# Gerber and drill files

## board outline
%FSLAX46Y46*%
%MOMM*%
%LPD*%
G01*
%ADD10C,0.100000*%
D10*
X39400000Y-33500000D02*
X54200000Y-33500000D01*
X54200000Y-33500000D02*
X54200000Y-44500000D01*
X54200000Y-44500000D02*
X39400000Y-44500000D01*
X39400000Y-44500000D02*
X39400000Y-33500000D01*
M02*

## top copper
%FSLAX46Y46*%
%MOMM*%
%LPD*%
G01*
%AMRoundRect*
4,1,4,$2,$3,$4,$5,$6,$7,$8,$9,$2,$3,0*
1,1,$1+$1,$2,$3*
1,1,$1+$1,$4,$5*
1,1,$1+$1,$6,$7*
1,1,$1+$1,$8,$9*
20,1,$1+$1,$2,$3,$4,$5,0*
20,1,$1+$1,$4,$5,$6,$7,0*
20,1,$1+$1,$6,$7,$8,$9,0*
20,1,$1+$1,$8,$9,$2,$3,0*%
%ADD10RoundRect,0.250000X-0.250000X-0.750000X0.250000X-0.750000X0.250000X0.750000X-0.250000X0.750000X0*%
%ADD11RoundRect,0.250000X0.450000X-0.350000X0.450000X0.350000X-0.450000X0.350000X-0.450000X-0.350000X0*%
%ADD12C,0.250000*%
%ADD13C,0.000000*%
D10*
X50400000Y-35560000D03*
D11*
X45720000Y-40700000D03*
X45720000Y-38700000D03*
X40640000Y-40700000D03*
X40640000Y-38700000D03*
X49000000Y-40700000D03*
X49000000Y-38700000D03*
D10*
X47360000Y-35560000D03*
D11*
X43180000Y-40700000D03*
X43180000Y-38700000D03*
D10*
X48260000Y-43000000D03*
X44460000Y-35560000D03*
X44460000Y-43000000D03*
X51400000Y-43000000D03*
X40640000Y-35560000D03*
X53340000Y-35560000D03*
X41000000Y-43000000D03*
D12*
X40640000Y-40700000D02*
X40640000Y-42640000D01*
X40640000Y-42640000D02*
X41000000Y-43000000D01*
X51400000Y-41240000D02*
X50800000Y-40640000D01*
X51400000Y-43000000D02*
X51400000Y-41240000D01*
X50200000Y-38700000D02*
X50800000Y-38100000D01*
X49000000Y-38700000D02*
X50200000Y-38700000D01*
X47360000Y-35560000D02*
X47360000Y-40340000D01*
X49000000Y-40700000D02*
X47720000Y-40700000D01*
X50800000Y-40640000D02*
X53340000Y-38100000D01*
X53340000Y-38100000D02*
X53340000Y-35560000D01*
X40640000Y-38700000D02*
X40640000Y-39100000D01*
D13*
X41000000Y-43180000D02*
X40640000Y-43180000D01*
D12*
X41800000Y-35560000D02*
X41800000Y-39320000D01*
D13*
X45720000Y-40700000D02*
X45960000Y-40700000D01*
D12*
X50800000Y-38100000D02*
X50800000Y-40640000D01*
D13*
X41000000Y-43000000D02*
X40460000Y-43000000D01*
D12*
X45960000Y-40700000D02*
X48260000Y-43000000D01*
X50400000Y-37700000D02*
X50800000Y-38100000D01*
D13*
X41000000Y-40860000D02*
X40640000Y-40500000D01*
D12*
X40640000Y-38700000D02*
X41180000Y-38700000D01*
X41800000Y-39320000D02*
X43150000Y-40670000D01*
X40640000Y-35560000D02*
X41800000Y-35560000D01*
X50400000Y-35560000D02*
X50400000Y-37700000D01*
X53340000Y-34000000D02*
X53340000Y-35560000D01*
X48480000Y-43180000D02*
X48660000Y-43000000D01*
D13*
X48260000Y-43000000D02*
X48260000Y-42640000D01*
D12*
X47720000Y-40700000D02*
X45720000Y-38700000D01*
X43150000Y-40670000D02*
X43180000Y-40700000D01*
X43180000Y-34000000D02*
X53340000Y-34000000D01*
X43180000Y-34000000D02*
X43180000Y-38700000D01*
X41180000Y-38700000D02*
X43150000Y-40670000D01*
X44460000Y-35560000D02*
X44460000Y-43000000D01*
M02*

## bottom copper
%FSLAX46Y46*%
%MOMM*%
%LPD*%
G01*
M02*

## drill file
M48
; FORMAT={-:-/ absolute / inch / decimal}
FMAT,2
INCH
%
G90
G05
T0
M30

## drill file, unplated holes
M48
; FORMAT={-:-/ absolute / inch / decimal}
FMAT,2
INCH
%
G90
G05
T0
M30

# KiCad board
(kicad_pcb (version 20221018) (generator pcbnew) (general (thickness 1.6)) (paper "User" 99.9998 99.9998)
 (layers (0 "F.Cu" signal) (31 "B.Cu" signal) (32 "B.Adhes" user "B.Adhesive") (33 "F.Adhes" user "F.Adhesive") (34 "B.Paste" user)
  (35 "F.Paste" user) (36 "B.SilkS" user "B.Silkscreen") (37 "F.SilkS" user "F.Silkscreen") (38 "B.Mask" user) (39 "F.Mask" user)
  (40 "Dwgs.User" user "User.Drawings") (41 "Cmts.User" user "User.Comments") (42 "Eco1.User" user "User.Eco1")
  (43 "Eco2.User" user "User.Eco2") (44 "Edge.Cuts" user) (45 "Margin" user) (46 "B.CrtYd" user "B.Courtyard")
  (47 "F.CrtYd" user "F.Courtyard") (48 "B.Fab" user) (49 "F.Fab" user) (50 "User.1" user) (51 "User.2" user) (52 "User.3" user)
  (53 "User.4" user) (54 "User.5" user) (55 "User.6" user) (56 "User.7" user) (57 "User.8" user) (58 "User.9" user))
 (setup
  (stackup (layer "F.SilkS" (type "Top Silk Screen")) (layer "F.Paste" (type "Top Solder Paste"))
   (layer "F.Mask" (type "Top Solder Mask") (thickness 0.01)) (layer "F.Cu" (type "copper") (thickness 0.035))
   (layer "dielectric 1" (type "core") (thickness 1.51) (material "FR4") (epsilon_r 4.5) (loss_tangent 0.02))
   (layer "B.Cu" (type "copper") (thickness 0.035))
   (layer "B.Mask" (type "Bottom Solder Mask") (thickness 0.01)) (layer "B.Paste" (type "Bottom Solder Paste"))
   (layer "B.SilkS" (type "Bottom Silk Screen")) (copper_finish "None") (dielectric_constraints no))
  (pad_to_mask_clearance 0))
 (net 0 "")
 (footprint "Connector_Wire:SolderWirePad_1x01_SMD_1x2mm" (layer "F.Cu") (at 50.4 35.56)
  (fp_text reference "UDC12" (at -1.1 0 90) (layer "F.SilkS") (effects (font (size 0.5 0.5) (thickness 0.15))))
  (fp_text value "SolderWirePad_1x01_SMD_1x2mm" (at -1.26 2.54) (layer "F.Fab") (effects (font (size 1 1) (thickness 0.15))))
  (pad "1" smd roundrect (at 0 0) (size 1 2) (layers "F.Cu" "F.Paste" "F.Mask") (roundrect_rratio 0.25)))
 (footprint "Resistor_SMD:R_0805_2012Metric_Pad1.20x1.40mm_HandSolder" (layer "F.Cu") (at 45.72 39.7 90)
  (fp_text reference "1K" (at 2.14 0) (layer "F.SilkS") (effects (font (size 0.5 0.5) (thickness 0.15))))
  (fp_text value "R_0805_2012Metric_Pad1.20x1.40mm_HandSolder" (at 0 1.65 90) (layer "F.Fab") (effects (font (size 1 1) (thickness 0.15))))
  (pad "1" smd roundrect (at -1 0 90) (size 1.2 1.4) (layers "F.Cu" "F.Paste" "F.Mask") (roundrect_rratio 0.2083333333))
  (pad "2" smd roundrect (at 1 0 90) (size 1.2 1.4) (layers "F.Cu" "F.Paste" "F.Mask") (roundrect_rratio 0.2083333333)))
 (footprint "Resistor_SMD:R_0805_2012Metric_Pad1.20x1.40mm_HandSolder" (layer "F.Cu") (at 40.64 39.7 90)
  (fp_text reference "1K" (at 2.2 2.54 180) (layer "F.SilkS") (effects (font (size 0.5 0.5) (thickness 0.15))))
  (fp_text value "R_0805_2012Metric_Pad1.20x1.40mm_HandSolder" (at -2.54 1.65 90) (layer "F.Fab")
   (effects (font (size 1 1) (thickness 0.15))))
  (pad "1" smd roundrect (at -1 0 90) (size 1.2 1.4) (layers "F.Cu" "F.Paste" "F.Mask") (roundrect_rratio 0.2083333333))
  (pad "2" smd roundrect (at 1 0 90) (size 1.2 1.4) (layers "F.Cu" "F.Paste" "F.Mask") (roundrect_rratio 0.2083333333)))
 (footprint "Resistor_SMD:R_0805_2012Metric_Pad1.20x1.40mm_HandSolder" (layer "F.Cu") (at 49 39.7 90)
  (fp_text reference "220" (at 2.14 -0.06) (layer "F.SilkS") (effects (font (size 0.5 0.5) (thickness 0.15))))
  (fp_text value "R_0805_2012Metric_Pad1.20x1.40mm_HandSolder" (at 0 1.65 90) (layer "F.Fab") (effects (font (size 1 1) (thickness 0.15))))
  (pad "1" smd roundrect (at -1 0 90) (size 1.2 1.4) (layers "F.Cu" "F.Paste" "F.Mask") (roundrect_rratio 0.2083333333))
  (pad "2" smd roundrect (at 1 0 90) (size 1.2 1.4) (layers "F.Cu" "F.Paste" "F.Mask") (roundrect_rratio 0.2083333333)))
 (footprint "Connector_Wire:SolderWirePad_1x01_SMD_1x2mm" (layer "F.Cu") (at 47.36 35.56)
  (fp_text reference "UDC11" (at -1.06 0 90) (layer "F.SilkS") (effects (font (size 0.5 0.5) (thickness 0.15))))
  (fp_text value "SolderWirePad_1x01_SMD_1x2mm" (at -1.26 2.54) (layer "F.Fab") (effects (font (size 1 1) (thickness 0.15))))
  (pad "1" smd roundrect (at 0 0) (size 1 2) (layers "F.Cu" "F.Paste" "F.Mask") (roundrect_rratio 0.25)))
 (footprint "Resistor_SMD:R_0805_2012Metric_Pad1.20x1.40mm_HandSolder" (layer "F.Cu") (at 43.18 39.7 90)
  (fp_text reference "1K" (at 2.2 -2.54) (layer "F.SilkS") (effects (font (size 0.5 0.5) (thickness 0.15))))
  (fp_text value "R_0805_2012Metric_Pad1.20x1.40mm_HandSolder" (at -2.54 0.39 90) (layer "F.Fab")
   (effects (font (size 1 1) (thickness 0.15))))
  (pad "1" smd roundrect (at -1 0 90) (size 1.2 1.4) (layers "F.Cu" "F.Paste" "F.Mask") (roundrect_rratio 0.2083333333))
  (pad "2" smd roundrect (at 1 0 90) (size 1.2 1.4) (layers "F.Cu" "F.Paste" "F.Mask") (roundrect_rratio 0.2083333333)))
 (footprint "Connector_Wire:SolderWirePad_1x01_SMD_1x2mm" (layer "F.Cu") (at 48.26 43)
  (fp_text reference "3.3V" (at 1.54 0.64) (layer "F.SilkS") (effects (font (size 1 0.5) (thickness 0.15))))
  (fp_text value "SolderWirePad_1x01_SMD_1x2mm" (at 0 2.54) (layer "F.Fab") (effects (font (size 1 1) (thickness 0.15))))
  (pad "1" smd roundrect (at 0 0) (size 1 2) (layers "F.Cu" "F.Paste" "F.Mask") (roundrect_rratio 0.25)))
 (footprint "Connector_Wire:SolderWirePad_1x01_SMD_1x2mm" (layer "F.Cu") (at 44.46 35.56)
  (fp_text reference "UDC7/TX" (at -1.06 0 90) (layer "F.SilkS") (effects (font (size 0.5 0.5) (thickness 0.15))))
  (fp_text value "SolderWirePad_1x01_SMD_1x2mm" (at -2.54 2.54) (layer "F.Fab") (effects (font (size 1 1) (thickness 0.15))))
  (pad "1" smd roundrect (at 0 0) (size 1 2) (layers "F.Cu" "F.Paste" "F.Mask") (roundrect_rratio 0.25)))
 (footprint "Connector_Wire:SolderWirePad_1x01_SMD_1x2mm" (layer "F.Cu") (at 44.46 43)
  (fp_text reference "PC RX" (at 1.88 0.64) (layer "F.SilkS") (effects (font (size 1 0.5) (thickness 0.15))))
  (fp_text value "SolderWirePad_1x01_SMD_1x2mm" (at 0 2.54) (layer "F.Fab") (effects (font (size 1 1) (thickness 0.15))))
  (pad "1" smd roundrect (at 0 0) (size 1 2) (layers "F.Cu" "F.Paste" "F.Mask") (roundrect_rratio 0.25)))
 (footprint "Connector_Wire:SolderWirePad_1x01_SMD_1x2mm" (layer "F.Cu") (at 51.4 43)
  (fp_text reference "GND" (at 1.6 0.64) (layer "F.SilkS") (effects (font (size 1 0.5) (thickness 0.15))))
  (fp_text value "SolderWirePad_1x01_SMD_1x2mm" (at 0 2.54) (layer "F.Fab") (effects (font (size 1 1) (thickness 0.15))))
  (pad "1" smd roundrect (at 0 0) (size 1 2) (layers "F.Cu" "F.Paste" "F.Mask") (roundrect_rratio 0.25)))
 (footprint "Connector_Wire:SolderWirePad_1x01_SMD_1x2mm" (layer "F.Cu") (at 40.64 35.56)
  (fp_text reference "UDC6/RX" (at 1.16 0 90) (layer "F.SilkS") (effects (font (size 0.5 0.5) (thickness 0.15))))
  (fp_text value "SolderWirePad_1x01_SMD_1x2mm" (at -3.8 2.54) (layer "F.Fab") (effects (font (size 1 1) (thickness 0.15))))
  (pad "1" smd roundrect (at 0 0) (size 1 2) (layers "F.Cu" "F.Paste" "F.Mask") (roundrect_rratio 0.25)))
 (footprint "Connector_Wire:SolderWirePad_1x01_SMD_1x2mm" (layer "F.Cu") (at 53.34 35.56)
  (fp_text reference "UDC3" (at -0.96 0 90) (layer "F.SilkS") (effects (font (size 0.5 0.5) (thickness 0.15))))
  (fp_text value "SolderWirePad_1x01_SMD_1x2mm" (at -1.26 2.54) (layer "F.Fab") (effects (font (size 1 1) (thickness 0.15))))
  (pad "1" smd roundrect (at 0 0) (size 1 2) (layers "F.Cu" "F.Paste" "F.Mask") (roundrect_rratio 0.25)))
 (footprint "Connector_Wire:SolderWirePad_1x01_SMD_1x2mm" (layer "F.Cu") (at 41 43)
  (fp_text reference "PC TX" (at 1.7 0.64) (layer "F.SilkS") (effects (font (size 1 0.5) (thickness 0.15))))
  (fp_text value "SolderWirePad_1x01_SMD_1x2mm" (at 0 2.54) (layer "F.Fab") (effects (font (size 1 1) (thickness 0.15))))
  (pad "1" smd roundrect (at 0 0) (size 1 2) (layers "F.Cu" "F.Paste" "F.Mask") (roundrect_rratio 0.25)))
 (gr_rect (start 39.4 33.5) (end 54.2 44.5) (stroke (width 0.1) (type default)) (fill none) (layer "Edge.Cuts"))
 (segment (start 51.4 43) (end 51.4 41.24) (width 0.25) (layer "F.Cu") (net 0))
 (segment (start 47.36 35.56) (end 47.36 40.34) (width 0.25) (layer "F.Cu") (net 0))
 (segment (start 49 40.7) (end 47.72 40.7) (width 0.25) (layer "F.Cu") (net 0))
 (segment (start 50.8 40.64) (end 53.34 38.1) (width 0.25) (layer "F.Cu") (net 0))
 (segment (start 40.64 40.7) (end 40.64 42.64) (width 0.25) (layer "F.Cu") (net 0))
 (segment (start 53.34 38.1) (end 53.34 35.56) (width 0.25) (layer "F.Cu") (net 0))
 (segment (start 40.64 38.7) (end 40.64 39.1) (width 0.25) (layer "F.Cu") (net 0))
 (segment (start 41 43.18) (end 40.64 43.18) (width 0) (layer "F.Cu") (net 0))
 (segment (start 41.8 35.56) (end 41.8 39.32) (width 0.25) (layer "F.Cu") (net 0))
 (segment (start 45.72 40.7) (end 45.96 40.7) (width 0) (layer "F.Cu") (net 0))
 (segment (start 50.8 38.1) (end 50.8 40.64) (width 0.25) (layer "F.Cu") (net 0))
 (segment (start 41 43) (end 40.46 43) (width 0) (layer "F.Cu") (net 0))
 (segment (start 40.64 42.64) (end 41 43) (width 0.25) (layer "F.Cu") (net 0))
 (segment (start 45.96 40.7) (end 48.26 43) (width 0.25) (layer "F.Cu") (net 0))
 (segment (start 50.4 37.7) (end 50.8 38.1) (width 0.25) (layer "F.Cu") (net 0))
 (segment (start 50.2 38.7) (end 50.8 38.1) (width 0.25) (layer "F.Cu") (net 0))
 (segment (start 41 40.86) (end 40.64 40.5) (width 0) (layer "F.Cu") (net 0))
 (segment (start 40.64 38.7) (end 41.18 38.7) (width 0.25) (layer "F.Cu") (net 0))
 (segment (start 41.8 39.32) (end 43.15 40.67) (width 0.25) (layer "F.Cu") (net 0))
 (segment (start 51.4 41.24) (end 50.8 40.64) (width 0.25) (layer "F.Cu") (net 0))
 (segment (start 40.64 35.56) (end 41.8 35.56) (width 0.25) (layer "F.Cu") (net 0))
 (segment (start 50.4 35.56) (end 50.4 37.7) (width 0.25) (layer "F.Cu") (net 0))
 (segment (start 53.34 34) (end 53.34 35.56) (width 0.25) (layer "F.Cu") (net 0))
 (segment (start 49 38.7) (end 50.2 38.7) (width 0.25) (layer "F.Cu") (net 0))
 (segment (start 48.48 43.18) (end 48.66 43) (width 0.25) (layer "F.Cu") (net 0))
 (segment (start 48.26 43) (end 48.26 42.64) (width 0) (layer "F.Cu") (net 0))
 (segment (start 47.72 40.7) (end 45.72 38.7) (width 0.25) (layer "F.Cu") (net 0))
 (segment (start 43.15 40.67) (end 43.18 40.7) (width 0.25) (layer "F.Cu") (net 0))
 (segment (start 43.18 34) (end 53.34 34) (width 0.25) (layer "F.Cu") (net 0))
 (segment (start 43.18 34) (end 43.18 38.7) (width 0.25) (layer "F.Cu") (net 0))
 (segment (start 41.18 38.7) (end 43.15 40.67) (width 0.25) (layer "F.Cu") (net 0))
 (segment (start 44.46 35.56) (end 44.46 43) (width 0.25) (layer "F.Cu") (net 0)))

